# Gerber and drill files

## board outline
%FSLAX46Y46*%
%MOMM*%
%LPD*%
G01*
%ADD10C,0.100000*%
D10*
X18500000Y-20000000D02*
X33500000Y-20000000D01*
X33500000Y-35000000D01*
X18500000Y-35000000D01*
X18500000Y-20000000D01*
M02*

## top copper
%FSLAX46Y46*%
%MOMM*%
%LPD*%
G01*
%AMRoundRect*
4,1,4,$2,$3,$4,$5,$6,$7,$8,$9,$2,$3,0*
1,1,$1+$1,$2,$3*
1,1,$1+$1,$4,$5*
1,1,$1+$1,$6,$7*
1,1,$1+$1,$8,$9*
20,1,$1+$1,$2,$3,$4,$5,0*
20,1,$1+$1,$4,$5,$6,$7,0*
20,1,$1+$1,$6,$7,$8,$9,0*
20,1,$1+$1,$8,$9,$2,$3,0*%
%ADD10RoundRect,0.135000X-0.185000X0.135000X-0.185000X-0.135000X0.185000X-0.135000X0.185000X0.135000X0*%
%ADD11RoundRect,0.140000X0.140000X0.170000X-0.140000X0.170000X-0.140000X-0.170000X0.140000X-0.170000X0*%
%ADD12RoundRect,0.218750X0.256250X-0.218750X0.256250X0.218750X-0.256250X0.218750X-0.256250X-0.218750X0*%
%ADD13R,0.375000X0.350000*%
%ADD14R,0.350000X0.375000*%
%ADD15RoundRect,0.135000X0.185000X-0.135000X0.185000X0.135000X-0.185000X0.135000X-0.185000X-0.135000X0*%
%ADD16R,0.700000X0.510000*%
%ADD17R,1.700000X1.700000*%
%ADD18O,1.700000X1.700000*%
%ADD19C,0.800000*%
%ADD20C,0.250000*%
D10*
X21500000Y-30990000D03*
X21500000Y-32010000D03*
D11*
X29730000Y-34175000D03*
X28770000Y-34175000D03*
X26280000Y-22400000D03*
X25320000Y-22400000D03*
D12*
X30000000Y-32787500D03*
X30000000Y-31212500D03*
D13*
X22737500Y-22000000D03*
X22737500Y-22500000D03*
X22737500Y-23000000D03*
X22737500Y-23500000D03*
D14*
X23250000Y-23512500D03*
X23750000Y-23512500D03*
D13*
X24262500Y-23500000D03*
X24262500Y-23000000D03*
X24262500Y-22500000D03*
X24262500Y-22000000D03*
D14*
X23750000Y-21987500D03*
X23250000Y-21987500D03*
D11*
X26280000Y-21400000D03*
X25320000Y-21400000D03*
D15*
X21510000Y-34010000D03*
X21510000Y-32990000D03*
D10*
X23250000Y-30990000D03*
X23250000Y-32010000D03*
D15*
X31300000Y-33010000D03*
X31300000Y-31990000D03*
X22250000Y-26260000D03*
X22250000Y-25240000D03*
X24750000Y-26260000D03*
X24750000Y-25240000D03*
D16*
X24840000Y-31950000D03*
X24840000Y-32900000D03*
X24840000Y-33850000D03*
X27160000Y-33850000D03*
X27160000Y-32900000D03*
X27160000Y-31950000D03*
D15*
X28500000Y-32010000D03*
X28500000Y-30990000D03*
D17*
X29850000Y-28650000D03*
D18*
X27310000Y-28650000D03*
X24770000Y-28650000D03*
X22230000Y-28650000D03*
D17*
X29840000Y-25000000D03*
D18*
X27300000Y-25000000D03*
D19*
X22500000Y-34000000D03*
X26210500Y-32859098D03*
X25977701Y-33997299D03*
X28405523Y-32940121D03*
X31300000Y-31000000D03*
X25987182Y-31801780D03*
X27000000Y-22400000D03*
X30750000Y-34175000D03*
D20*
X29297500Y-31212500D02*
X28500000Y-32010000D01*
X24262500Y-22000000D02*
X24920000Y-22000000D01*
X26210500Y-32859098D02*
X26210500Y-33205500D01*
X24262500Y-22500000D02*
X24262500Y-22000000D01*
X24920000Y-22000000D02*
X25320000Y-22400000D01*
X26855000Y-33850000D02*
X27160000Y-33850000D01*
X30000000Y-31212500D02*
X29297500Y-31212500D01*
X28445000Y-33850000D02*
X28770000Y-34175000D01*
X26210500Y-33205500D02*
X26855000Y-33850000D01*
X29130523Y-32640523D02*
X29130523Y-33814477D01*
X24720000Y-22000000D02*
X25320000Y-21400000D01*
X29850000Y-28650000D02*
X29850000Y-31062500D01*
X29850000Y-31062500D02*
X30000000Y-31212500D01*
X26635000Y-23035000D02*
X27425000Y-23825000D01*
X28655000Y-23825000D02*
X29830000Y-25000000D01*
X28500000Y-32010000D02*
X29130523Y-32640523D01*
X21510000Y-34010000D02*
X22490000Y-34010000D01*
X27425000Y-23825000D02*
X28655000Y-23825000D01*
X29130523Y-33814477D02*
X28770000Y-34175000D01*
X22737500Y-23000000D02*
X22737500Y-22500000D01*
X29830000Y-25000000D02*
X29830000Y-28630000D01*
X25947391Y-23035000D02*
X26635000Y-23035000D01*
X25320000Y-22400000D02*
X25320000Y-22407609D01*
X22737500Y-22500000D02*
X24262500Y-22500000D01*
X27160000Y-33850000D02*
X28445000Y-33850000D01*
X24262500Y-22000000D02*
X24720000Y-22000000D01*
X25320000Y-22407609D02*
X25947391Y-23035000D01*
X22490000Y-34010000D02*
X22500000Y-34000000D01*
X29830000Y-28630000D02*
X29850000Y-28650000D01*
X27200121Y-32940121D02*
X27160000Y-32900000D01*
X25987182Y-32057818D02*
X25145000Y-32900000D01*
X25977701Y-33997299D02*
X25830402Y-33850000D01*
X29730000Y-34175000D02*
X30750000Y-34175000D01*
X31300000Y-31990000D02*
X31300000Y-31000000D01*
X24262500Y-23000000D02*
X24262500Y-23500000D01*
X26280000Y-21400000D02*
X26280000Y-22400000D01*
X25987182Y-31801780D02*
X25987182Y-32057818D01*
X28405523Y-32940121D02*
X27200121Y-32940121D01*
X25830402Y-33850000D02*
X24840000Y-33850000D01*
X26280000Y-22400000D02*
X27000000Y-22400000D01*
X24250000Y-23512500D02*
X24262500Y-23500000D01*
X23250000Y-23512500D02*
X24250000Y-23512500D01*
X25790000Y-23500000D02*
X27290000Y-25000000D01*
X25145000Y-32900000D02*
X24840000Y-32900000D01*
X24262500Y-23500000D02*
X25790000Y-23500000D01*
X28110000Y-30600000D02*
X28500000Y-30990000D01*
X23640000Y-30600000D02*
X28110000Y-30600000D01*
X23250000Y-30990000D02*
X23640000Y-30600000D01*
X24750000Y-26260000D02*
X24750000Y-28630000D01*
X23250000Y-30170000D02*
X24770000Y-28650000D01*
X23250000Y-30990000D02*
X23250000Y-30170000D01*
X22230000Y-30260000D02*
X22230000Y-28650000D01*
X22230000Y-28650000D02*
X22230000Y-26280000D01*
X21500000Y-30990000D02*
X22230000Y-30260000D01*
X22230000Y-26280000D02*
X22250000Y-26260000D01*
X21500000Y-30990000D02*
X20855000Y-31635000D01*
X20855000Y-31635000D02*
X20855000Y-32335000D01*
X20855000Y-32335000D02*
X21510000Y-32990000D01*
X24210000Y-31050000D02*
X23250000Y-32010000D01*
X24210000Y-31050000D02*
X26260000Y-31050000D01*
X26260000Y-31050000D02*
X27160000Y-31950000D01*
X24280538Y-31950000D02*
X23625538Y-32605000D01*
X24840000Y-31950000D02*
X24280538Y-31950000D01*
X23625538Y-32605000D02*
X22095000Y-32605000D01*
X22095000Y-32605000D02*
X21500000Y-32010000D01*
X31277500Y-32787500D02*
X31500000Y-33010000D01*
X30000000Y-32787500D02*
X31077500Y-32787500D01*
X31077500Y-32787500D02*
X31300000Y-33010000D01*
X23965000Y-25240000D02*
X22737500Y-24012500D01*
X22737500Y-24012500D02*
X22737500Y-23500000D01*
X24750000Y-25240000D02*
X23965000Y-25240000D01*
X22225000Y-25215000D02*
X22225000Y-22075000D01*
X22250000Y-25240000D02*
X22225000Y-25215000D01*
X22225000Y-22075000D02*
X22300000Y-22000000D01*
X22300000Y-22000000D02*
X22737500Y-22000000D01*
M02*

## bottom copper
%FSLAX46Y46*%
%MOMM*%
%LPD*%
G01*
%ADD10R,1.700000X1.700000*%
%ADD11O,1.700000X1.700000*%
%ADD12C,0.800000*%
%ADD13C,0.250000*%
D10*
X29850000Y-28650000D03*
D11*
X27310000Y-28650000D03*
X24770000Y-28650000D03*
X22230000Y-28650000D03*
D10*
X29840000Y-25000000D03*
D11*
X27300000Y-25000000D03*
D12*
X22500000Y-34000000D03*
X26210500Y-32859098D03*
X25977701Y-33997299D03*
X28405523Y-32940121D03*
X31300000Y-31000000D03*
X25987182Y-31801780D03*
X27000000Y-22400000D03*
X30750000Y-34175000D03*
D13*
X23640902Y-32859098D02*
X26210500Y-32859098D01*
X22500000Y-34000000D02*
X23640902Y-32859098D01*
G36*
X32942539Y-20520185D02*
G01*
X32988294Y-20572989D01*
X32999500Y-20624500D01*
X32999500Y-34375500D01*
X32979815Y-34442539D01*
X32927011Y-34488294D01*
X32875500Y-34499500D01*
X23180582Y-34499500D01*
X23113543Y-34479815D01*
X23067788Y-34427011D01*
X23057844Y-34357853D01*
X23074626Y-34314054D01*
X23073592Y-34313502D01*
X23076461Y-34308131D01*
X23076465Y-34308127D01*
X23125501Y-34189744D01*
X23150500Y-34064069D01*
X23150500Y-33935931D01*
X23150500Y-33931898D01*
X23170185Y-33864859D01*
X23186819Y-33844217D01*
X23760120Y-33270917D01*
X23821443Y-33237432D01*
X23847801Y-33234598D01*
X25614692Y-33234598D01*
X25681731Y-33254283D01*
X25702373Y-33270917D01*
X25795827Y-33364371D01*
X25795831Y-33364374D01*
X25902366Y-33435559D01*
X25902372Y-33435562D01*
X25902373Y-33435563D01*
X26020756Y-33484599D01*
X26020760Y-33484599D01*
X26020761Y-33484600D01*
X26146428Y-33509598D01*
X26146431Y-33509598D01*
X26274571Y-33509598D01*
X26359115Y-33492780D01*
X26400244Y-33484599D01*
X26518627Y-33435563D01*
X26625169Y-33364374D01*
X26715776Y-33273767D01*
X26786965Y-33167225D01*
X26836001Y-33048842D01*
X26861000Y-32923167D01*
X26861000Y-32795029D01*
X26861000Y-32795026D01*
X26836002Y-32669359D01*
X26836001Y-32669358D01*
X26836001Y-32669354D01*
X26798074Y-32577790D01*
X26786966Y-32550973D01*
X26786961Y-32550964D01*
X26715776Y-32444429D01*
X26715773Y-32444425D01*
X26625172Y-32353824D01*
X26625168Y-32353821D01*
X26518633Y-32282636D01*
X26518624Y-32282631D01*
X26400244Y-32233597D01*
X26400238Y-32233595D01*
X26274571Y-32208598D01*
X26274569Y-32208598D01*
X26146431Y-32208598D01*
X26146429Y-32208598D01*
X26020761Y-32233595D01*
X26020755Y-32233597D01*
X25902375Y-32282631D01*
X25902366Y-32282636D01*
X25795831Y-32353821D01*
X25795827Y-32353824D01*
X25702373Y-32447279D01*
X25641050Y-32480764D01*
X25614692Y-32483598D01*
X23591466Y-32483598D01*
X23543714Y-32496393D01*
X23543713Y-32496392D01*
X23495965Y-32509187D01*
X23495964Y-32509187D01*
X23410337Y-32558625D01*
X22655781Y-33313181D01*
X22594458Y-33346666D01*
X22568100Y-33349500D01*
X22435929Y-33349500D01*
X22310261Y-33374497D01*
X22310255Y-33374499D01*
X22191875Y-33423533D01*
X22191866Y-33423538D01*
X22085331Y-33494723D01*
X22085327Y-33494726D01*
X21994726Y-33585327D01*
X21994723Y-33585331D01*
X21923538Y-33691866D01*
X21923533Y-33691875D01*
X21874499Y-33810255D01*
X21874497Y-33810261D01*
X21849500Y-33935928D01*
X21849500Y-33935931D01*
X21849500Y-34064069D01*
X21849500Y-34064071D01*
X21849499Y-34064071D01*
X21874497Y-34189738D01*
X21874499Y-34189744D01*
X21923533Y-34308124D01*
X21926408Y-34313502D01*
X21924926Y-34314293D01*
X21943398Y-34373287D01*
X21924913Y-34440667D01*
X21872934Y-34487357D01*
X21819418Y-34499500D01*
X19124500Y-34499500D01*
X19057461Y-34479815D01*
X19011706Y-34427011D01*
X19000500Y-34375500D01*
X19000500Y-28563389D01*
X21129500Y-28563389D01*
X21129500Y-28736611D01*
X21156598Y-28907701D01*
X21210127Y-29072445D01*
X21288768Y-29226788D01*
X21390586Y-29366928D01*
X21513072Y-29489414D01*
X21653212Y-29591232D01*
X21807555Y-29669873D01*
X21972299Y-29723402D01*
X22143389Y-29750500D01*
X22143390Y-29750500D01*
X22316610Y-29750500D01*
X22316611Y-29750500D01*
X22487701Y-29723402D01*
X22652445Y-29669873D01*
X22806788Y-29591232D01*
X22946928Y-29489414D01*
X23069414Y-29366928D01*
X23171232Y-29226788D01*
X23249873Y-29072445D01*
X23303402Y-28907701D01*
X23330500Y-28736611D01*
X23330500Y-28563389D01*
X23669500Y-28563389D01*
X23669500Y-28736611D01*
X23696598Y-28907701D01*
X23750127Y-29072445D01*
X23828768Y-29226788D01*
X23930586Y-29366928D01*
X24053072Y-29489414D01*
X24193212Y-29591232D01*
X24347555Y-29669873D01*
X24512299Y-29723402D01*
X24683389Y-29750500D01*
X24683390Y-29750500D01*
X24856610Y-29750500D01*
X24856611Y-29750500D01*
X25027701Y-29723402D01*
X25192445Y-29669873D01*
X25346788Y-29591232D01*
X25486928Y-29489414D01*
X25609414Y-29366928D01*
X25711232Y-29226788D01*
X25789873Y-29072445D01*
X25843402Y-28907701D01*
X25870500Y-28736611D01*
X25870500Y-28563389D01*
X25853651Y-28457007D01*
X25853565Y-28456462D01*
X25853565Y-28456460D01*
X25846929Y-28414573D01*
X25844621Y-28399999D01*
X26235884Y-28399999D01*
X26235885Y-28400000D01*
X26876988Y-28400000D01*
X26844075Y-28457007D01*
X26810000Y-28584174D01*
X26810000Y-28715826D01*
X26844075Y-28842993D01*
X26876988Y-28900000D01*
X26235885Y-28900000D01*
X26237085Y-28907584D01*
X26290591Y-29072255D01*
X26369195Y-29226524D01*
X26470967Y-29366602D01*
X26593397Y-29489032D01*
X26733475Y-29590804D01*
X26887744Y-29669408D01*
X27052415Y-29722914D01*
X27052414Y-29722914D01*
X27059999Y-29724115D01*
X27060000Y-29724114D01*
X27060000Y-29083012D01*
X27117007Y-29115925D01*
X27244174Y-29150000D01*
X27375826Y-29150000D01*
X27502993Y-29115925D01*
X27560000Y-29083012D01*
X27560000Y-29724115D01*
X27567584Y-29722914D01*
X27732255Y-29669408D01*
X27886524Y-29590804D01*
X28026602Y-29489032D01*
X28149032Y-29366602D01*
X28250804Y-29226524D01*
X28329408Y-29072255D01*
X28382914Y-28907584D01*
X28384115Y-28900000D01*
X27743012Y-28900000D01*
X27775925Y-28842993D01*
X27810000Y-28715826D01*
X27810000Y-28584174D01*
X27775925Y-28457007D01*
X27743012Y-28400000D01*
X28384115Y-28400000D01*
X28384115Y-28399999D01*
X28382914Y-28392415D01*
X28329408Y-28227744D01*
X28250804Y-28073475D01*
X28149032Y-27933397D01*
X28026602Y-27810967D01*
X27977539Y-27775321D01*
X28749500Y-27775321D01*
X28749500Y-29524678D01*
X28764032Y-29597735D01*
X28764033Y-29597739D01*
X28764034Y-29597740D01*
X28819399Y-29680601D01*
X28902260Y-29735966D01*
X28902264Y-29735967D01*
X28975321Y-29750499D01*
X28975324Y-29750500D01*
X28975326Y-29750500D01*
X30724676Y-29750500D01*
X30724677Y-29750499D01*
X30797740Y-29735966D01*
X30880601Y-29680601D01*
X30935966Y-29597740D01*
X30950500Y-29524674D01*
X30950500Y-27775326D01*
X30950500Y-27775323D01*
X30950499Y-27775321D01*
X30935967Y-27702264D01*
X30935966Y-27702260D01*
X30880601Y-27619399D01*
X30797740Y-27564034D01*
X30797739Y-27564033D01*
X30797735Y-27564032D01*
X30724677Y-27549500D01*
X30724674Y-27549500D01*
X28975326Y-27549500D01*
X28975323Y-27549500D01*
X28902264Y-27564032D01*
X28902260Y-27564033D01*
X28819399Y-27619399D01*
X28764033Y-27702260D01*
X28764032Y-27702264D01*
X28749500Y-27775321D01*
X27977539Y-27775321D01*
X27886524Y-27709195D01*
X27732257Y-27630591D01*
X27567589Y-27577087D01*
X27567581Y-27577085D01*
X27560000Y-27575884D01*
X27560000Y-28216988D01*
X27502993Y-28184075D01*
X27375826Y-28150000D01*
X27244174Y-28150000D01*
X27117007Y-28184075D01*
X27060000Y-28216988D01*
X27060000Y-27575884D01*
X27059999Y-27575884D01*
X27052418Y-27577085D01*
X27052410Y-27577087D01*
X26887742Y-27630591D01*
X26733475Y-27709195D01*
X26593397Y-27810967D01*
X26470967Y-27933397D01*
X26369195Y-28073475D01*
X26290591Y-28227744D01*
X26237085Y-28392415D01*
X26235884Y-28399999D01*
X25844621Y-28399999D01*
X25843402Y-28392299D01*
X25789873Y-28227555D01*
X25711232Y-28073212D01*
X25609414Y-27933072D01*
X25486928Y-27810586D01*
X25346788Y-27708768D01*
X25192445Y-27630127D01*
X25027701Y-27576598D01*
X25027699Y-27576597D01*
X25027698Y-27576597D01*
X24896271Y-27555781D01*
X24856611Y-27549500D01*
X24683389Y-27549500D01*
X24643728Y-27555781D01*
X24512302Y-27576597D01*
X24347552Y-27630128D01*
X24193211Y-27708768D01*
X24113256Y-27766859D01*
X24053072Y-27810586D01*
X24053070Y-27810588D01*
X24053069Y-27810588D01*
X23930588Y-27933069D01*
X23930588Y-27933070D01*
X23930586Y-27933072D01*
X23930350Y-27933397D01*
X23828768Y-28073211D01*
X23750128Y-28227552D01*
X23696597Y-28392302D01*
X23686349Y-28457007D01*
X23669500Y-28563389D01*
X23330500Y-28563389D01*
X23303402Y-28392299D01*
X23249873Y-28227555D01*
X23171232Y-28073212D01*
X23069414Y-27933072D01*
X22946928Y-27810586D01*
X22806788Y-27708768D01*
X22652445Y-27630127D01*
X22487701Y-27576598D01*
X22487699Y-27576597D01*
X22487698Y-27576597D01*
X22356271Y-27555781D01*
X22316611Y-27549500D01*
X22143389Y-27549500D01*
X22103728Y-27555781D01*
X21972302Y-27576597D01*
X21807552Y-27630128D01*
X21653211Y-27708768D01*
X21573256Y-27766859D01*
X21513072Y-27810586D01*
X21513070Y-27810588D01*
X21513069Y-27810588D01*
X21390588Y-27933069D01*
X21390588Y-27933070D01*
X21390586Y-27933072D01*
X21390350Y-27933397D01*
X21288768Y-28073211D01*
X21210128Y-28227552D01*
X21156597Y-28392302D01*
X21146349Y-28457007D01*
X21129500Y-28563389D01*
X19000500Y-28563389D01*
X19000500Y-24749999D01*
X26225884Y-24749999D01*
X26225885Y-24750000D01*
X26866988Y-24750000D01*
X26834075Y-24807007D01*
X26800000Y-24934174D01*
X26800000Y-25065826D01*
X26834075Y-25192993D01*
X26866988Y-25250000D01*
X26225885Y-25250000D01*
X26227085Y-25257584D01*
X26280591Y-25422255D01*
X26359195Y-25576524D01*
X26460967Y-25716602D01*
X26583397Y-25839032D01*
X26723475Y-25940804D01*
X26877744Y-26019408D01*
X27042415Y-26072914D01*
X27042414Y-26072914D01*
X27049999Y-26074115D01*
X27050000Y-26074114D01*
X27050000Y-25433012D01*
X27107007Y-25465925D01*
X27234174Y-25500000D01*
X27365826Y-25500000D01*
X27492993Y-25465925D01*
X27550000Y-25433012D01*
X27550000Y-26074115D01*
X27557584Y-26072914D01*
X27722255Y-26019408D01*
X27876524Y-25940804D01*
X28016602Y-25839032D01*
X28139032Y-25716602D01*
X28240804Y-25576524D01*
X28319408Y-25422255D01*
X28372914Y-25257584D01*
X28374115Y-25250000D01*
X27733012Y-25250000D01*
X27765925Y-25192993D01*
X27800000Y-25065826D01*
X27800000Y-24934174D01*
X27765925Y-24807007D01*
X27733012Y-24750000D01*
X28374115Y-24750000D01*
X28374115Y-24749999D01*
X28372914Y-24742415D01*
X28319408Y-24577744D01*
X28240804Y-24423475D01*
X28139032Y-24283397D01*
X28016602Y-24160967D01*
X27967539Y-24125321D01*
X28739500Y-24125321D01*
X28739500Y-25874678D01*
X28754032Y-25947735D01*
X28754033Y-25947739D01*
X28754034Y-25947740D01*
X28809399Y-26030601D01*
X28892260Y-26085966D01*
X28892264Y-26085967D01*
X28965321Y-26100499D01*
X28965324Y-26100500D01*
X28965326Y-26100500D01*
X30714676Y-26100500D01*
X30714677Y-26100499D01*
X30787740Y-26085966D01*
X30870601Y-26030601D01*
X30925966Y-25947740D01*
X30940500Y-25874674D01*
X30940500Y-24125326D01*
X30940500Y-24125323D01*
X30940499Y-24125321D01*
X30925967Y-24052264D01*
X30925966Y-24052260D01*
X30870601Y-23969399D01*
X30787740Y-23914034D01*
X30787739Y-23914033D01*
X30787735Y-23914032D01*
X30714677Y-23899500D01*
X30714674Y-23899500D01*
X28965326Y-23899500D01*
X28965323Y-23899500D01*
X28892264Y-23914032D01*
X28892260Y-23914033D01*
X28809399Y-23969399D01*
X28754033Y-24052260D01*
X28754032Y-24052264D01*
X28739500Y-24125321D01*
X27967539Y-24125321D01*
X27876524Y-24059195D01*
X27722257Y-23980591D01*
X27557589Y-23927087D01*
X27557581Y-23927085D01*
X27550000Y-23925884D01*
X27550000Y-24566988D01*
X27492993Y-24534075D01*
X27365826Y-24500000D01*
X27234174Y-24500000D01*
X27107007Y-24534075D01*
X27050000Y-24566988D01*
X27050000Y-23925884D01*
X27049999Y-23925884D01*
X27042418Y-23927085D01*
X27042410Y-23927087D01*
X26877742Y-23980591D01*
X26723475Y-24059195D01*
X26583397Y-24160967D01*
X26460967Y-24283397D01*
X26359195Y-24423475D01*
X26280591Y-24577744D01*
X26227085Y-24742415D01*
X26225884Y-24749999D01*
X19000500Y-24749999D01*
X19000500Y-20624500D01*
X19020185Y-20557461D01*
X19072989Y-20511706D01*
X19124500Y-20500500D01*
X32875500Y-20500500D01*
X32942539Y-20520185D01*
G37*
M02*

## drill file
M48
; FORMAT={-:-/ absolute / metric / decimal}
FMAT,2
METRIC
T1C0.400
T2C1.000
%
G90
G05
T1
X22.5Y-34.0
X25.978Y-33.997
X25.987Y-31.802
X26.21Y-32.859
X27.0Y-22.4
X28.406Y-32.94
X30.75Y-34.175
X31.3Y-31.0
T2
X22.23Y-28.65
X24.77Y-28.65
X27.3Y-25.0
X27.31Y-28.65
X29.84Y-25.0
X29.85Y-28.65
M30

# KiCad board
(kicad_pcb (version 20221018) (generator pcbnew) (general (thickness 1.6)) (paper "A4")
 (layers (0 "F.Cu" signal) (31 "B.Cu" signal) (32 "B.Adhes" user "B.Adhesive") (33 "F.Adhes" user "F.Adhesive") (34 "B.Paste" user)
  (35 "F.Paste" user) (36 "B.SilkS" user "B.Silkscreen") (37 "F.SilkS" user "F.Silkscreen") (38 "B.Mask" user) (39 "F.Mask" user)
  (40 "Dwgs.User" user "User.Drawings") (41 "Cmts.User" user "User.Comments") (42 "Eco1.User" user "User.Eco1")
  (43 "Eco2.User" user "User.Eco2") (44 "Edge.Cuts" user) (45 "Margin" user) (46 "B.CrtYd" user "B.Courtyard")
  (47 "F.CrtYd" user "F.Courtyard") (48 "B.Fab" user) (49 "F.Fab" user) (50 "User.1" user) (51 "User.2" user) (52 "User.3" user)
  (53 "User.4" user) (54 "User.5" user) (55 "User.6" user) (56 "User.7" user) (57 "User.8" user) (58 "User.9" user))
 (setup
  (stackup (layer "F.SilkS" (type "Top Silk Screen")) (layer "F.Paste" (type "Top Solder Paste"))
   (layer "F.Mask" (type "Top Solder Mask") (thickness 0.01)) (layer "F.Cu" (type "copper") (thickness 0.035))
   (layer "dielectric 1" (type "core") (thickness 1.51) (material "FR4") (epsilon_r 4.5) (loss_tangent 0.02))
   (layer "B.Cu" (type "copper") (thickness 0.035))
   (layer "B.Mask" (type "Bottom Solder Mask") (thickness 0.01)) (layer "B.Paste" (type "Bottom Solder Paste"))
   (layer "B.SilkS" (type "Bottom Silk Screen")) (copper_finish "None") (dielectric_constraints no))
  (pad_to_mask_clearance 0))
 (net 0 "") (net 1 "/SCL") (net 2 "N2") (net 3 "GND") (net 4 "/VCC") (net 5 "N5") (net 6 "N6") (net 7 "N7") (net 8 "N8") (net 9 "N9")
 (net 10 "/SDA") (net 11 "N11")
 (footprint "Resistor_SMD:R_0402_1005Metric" (layer "F.Cu") (at 21.5 31.5 -90)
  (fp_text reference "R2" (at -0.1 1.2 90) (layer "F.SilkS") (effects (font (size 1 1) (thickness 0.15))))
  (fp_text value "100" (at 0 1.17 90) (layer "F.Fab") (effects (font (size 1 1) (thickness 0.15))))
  (pad "1" smd roundrect (at -0.51 0 270) (size 0.54 0.64) (layers "F.Cu" "F.Paste" "F.Mask") (roundrect_rratio 0.25) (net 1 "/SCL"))
  (pad "2" smd roundrect (at 0.51 0 270) (size 0.54 0.64) (layers "F.Cu" "F.Paste" "F.Mask") (roundrect_rratio 0.25) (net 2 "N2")))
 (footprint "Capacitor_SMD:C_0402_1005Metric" (layer "F.Cu") (at 29.25 34.175 180)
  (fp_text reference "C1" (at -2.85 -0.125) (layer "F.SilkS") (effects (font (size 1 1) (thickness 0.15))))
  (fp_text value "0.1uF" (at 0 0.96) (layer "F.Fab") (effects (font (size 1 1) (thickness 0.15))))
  (pad "1" smd roundrect (at -0.48 0 180) (size 0.56 0.62) (layers "F.Cu" "F.Paste" "F.Mask") (roundrect_rratio 0.25) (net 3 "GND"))
  (pad "2" smd roundrect (at 0.48 0 180) (size 0.56 0.62) (layers "F.Cu" "F.Paste" "F.Mask") (roundrect_rratio 0.25) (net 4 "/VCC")))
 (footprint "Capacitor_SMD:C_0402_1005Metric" (layer "F.Cu") (at 25.8 22.4 180)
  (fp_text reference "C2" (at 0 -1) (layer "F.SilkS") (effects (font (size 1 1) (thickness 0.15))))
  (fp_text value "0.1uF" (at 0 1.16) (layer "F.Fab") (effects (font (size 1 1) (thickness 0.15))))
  (pad "1" smd roundrect (at -0.48 0 180) (size 0.56 0.62) (layers "F.Cu" "F.Paste" "F.Mask") (roundrect_rratio 0.25) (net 3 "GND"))
  (pad "2" smd roundrect (at 0.48 0 180) (size 0.56 0.62) (layers "F.Cu" "F.Paste" "F.Mask") (roundrect_rratio 0.25) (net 4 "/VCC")))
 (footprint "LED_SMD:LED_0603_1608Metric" (layer "F.Cu") (at 30 32 90)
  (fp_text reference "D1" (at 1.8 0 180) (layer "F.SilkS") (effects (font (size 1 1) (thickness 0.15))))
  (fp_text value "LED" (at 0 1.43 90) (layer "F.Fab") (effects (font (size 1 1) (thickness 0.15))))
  (pad "1" smd roundrect (at -0.7875 0 90) (size 0.875 0.95) (layers "F.Cu" "F.Paste" "F.Mask") (roundrect_rratio 0.25) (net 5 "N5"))
  (pad "2" smd roundrect (at 0.7875 0 90) (size 0.875 0.95) (layers "F.Cu" "F.Paste" "F.Mask") (roundrect_rratio 0.25) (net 4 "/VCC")))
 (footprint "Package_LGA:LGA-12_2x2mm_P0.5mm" (layer "F.Cu") (at 23.5 22.75)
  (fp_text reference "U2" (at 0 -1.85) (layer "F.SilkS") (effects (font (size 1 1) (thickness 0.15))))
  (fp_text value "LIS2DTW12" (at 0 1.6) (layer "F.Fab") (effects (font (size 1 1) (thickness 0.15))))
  (pad "1" smd rect (at -0.7625 -0.75) (size 0.375 0.35) (layers "F.Cu" "F.Paste" "F.Mask") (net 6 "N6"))
  (pad "2" smd rect (at -0.7625 -0.25) (size 0.375 0.35) (layers "F.Cu" "F.Paste" "F.Mask") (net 4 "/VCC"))
  (pad "3" smd rect (at -0.7625 0.25) (size 0.375 0.35) (layers "F.Cu" "F.Paste" "F.Mask") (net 4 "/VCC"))
  (pad "4" smd rect (at -0.7625 0.75) (size 0.375 0.35) (layers "F.Cu" "F.Paste" "F.Mask") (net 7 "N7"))
  (pad "5" smd rect (at -0.25 0.7625 90) (size 0.375 0.35) (layers "F.Cu" "F.Paste" "F.Mask") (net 3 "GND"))
  (pad "6" smd rect (at 0.25 0.7625 90) (size 0.375 0.35) (layers "F.Cu" "F.Paste" "F.Mask") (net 3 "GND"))
  (pad "7" smd rect (at 0.7625 0.75) (size 0.375 0.35) (layers "F.Cu" "F.Paste" "F.Mask") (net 3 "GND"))
  (pad "8" smd rect (at 0.7625 0.25) (size 0.375 0.35) (layers "F.Cu" "F.Paste" "F.Mask") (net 3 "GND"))
  (pad "9" smd rect (at 0.7625 -0.25) (size 0.375 0.35) (layers "F.Cu" "F.Paste" "F.Mask") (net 4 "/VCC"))
  (pad "10" smd rect (at 0.7625 -0.75) (size 0.375 0.35) (layers "F.Cu" "F.Paste" "F.Mask") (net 4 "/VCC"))
  (pad "11" smd rect (at 0.25 -0.7625 90) (size 0.375 0.35) (layers "F.Cu" "F.Paste" "F.Mask") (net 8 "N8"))
  (pad "12" smd rect (at -0.25 -0.7625 90) (size 0.375 0.35) (layers "F.Cu" "F.Paste" "F.Mask") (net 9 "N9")))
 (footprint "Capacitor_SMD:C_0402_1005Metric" (layer "F.Cu") (at 25.8 21.4 180)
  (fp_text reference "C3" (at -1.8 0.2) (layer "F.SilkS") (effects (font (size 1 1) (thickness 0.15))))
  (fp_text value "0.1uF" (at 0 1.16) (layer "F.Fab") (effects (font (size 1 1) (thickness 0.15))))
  (pad "1" smd roundrect (at -0.48 0 180) (size 0.56 0.62) (layers "F.Cu" "F.Paste" "F.Mask") (roundrect_rratio 0.25) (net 3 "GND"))
  (pad "2" smd roundrect (at 0.48 0 180) (size 0.56 0.62) (layers "F.Cu" "F.Paste" "F.Mask") (roundrect_rratio 0.25) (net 4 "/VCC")))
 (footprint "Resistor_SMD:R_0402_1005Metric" (layer "F.Cu") (at 21.51 33.5 90)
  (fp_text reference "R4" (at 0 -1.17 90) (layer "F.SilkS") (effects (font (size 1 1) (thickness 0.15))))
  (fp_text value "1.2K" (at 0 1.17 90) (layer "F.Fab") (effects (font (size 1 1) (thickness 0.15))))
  (pad "1" smd roundrect (at -0.51 0 90) (size 0.54 0.64) (layers "F.Cu" "F.Paste" "F.Mask") (roundrect_rratio 0.25) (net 4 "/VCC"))
  (pad "2" smd roundrect (at 0.51 0 90) (size 0.54 0.64) (layers "F.Cu" "F.Paste" "F.Mask") (roundrect_rratio 0.25) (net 1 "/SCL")))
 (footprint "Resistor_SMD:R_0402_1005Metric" (layer "F.Cu") (at 23.25 31.5 -90)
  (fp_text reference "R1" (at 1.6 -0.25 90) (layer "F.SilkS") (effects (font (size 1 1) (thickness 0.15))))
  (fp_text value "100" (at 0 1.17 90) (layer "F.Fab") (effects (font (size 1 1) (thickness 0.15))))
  (pad "1" smd roundrect (at -0.51 0 270) (size 0.54 0.64) (layers "F.Cu" "F.Paste" "F.Mask") (roundrect_rratio 0.25) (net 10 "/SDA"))
  (pad "2" smd roundrect (at 0.51 0 270) (size 0.54 0.64) (layers "F.Cu" "F.Paste" "F.Mask") (roundrect_rratio 0.25) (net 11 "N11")))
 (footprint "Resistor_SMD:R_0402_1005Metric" (layer "F.Cu") (at 31.3 32.5 90)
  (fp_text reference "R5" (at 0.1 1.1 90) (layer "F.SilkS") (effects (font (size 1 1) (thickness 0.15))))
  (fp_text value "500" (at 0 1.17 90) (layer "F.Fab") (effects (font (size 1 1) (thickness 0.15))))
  (pad "1" smd roundrect (at -0.51 0 90) (size 0.54 0.64) (layers "F.Cu" "F.Paste" "F.Mask") (roundrect_rratio 0.25) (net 5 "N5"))
  (pad "2" smd roundrect (at 0.51 0 90) (size 0.54 0.64) (layers "F.Cu" "F.Paste" "F.Mask") (roundrect_rratio 0.25) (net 3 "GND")))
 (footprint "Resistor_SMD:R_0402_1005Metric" (layer "F.Cu") (at 22.25 25.75 90)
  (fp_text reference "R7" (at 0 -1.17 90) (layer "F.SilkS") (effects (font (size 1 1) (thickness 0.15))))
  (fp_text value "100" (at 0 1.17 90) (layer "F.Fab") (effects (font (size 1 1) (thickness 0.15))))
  (pad "1" smd roundrect (at -0.51 0 90) (size 0.54 0.64) (layers "F.Cu" "F.Paste" "F.Mask") (roundrect_rratio 0.25) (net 1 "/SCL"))
  (pad "2" smd roundrect (at 0.51 0 90) (size 0.54 0.64) (layers "F.Cu" "F.Paste" "F.Mask") (roundrect_rratio 0.25) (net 6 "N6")))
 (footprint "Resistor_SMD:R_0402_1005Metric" (layer "F.Cu") (at 24.75 25.75 90)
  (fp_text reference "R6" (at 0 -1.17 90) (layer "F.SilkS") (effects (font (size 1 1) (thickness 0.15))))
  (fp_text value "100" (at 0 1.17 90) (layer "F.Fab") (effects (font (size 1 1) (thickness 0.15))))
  (pad "1" smd roundrect (at -0.51 0 90) (size 0.54 0.64) (layers "F.Cu" "F.Paste" "F.Mask") (roundrect_rratio 0.25) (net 10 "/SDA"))
  (pad "2" smd roundrect (at 0.51 0 90) (size 0.54 0.64) (layers "F.Cu" "F.Paste" "F.Mask") (roundrect_rratio 0.25) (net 7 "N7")))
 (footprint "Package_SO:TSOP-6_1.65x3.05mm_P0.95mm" (layer "F.Cu") (at 26 32.9)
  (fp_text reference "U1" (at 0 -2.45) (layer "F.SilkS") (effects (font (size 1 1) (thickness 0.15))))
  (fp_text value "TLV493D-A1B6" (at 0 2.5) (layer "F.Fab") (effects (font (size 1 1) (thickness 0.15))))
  (pad "1" smd rect (at -1.16 -0.95) (size 0.7 0.51) (layers "F.Cu" "F.Paste" "F.Mask") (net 2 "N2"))
  (pad "2" smd rect (at -1.16 0) (size 0.7 0.51) (layers "F.Cu" "F.Paste" "F.Mask") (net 3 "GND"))
  (pad "3" smd rect (at -1.16 0.95) (size 0.7 0.51) (layers "F.Cu" "F.Paste" "F.Mask") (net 3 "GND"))
  (pad "4" smd rect (at 1.16 0.95) (size 0.7 0.51) (layers "F.Cu" "F.Paste" "F.Mask") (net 4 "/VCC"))
  (pad "5" smd rect (at 1.16 0) (size 0.7 0.51) (layers "F.Cu" "F.Paste" "F.Mask") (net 3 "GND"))
  (pad "6" smd rect (at 1.16 -0.95) (size 0.7 0.51) (layers "F.Cu" "F.Paste" "F.Mask") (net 11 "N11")))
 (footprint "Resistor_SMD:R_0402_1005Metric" (layer "F.Cu") (at 28.5 31.5 90)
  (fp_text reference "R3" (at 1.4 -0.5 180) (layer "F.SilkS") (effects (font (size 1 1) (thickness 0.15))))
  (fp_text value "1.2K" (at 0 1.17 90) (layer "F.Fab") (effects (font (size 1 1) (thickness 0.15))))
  (pad "1" smd roundrect (at -0.51 0 90) (size 0.54 0.64) (layers "F.Cu" "F.Paste" "F.Mask") (roundrect_rratio 0.25) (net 4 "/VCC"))
  (pad "2" smd roundrect (at 0.51 0 90) (size 0.54 0.64) (layers "F.Cu" "F.Paste" "F.Mask") (roundrect_rratio 0.25) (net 10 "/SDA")))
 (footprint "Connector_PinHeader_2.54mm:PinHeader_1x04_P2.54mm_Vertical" (layer "B.Cu") (at 29.85 28.65 90)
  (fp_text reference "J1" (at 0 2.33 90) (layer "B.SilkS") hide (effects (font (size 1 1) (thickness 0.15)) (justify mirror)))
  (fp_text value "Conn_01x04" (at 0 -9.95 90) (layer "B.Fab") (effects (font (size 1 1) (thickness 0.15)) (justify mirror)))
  (pad "1" thru_hole rect (at 0 0 90) (size 1.7 1.7) (drill 1) (layers "*.Cu" "*.Mask") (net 4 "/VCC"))
  (pad "2" thru_hole oval (at 0 -2.54 90) (size 1.7 1.7) (drill 1) (layers "*.Cu" "*.Mask") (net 3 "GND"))
  (pad "3" thru_hole oval (at 0 -5.08 90) (size 1.7 1.7) (drill 1) (layers "*.Cu" "*.Mask") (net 10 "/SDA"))
  (pad "4" thru_hole oval (at 0 -7.62 90) (size 1.7 1.7) (drill 1) (layers "*.Cu" "*.Mask") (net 1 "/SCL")))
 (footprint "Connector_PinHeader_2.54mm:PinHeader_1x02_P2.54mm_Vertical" (layer "B.Cu") (at 29.84 25 90)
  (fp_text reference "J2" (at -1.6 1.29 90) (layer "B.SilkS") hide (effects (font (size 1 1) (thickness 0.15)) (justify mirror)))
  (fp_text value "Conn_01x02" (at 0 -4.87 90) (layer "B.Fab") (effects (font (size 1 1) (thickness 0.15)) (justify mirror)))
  (pad "1" thru_hole rect (at 0 0 90) (size 1.7 1.7) (drill 1) (layers "*.Cu" "*.Mask") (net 4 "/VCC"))
  (pad "2" thru_hole oval (at 0 -2.54 90) (size 1.7 1.7) (drill 1) (layers "*.Cu" "*.Mask") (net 3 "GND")))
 (gr_rect (start 18.5 20) (end 33.5 35) (stroke (width 0.1) (type default)) (fill none) (layer "Edge.Cuts"))
 (segment (start 29.2975 31.2125) (end 28.5 32.01) (width 0.25) (layer "F.Cu") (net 4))
 (segment (start 24.2625 22) (end 24.92 22) (width 0.25) (layer "F.Cu") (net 4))
 (segment (start 26.2105 32.859098) (end 26.2105 33.2055) (width 0.25) (layer "F.Cu") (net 4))
 (segment (start 24.2625 22.5) (end 24.2625 22) (width 0.25) (layer "F.Cu") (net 4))
 (segment (start 24.92 22) (end 25.32 22.4) (width 0.25) (layer "F.Cu") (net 4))
 (segment (start 26.855 33.85) (end 27.16 33.85) (width 0.25) (layer "F.Cu") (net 4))
 (segment (start 30 31.2125) (end 29.2975 31.2125) (width 0.25) (layer "F.Cu") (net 4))
 (segment (start 28.445 33.85) (end 28.77 34.175) (width 0.25) (layer "F.Cu") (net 4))
 (segment (start 26.2105 33.2055) (end 26.855 33.85) (width 0.25) (layer "F.Cu") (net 4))
 (segment (start 29.130523 32.640523) (end 29.130523 33.814477) (width 0.25) (layer "F.Cu") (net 4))
 (segment (start 24.72 22) (end 25.32 21.4) (width 0.25) (layer "F.Cu") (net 4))
 (segment (start 29.85 28.65) (end 29.85 31.0625) (width 0.25) (layer "F.Cu") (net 4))
 (segment (start 29.85 31.0625) (end 30 31.2125) (width 0.25) (layer "F.Cu") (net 4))
 (segment (start 26.635 23.035) (end 27.425 23.825) (width 0.25) (layer "F.Cu") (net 4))
 (segment (start 28.655 23.825) (end 29.83 25) (width 0.25) (layer "F.Cu") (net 4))
 (segment (start 28.5 32.01) (end 29.130523 32.640523) (width 0.25) (layer "F.Cu") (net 4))
 (segment (start 21.51 34.01) (end 22.49 34.01) (width 0.25) (layer "F.Cu") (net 4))
 (segment (start 27.425 23.825) (end 28.655 23.825) (width 0.25) (layer "F.Cu") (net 4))
 (segment (start 29.130523 33.814477) (end 28.77 34.175) (width 0.25) (layer "F.Cu") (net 4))
 (segment (start 22.7375 23) (end 22.7375 22.5) (width 0.25) (layer "F.Cu") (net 4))
 (segment (start 29.83 25) (end 29.83 28.63) (width 0.25) (layer "F.Cu") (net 4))
 (segment (start 25.947391 23.035) (end 26.635 23.035) (width 0.25) (layer "F.Cu") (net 4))
 (segment (start 25.32 22.4) (end 25.32 22.407609) (width 0.25) (layer "F.Cu") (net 4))
 (segment (start 22.7375 22.5) (end 24.2625 22.5) (width 0.25) (layer "F.Cu") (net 4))
 (segment (start 27.16 33.85) (end 28.445 33.85) (width 0.25) (layer "F.Cu") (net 4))
 (segment (start 24.2625 22) (end 24.72 22) (width 0.25) (layer "F.Cu") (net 4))
 (segment (start 25.32 22.407609) (end 25.947391 23.035) (width 0.25) (layer "F.Cu") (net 4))
 (segment (start 22.49 34.01) (end 22.5 34) (width 0.25) (layer "F.Cu") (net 4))
 (segment (start 29.83 28.63) (end 29.85 28.65) (width 0.25) (layer "F.Cu") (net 4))
 (via (at 22.5 34) (size 0.8) (drill 0.4) (layers "F.Cu" "B.Cu") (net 4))
 (via (at 26.2105 32.859098) (size 0.8) (drill 0.4) (layers "F.Cu" "B.Cu") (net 4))
 (segment (start 23.640902 32.859098) (end 26.2105 32.859098) (width 0.25) (layer "B.Cu") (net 4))
 (segment (start 22.5 34) (end 23.640902 32.859098) (width 0.25) (layer "B.Cu") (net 4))
 (segment (start 27.200121 32.940121) (end 27.16 32.9) (width 0.25) (layer "F.Cu") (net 3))
 (segment (start 25.987182 32.057818) (end 25.145 32.9) (width 0.25) (layer "F.Cu") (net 3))
 (segment (start 25.977701 33.997299) (end 25.830402 33.85) (width 0.25) (layer "F.Cu") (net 3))
 (segment (start 29.73 34.175) (end 30.75 34.175) (width 0.25) (layer "F.Cu") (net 3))
 (segment (start 31.3 31.99) (end 31.3 31) (width 0.25) (layer "F.Cu") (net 3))
 (segment (start 24.2625 23) (end 24.2625 23.5) (width 0.25) (layer "F.Cu") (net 3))
 (segment (start 26.28 21.4) (end 26.28 22.4) (width 0.25) (layer "F.Cu") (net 3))
 (segment (start 25.987182 31.80178) (end 25.987182 32.057818) (width 0.25) (layer "F.Cu") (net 3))
 (segment (start 28.405523 32.940121) (end 27.200121 32.940121) (width 0.25) (layer "F.Cu") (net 3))
 (segment (start 25.830402 33.85) (end 24.84 33.85) (width 0.25) (layer "F.Cu") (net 3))
 (segment (start 26.28 22.4) (end 27 22.4) (width 0.25) (layer "F.Cu") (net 3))
 (segment (start 24.25 23.5125) (end 24.2625 23.5) (width 0.25) (layer "F.Cu") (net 3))
 (segment (start 23.25 23.5125) (end 24.25 23.5125) (width 0.25) (layer "F.Cu") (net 3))
 (segment (start 25.79 23.5) (end 27.29 25) (width 0.25) (layer "F.Cu") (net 3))
 (segment (start 25.145 32.9) (end 24.84 32.9) (width 0.25) (layer "F.Cu") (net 3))
 (segment (start 24.2625 23.5) (end 25.79 23.5) (width 0.25) (layer "F.Cu") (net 3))
 (via (at 25.977701 33.997299) (size 0.8) (drill 0.4) (layers "F.Cu" "B.Cu") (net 3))
 (via (at 28.405523 32.940121) (size 0.8) (drill 0.4) (layers "F.Cu" "B.Cu") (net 3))
 (via (at 31.3 31) (size 0.8) (drill 0.4) (layers "F.Cu" "B.Cu") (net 3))
 (via (at 25.987182 31.80178) (size 0.8) (drill 0.4) (layers "F.Cu" "B.Cu") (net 3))
 (via (at 27 22.4) (size 0.8) (drill 0.4) (layers "F.Cu" "B.Cu") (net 3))
 (via (at 30.75 34.175) (size 0.8) (drill 0.4) (layers "F.Cu" "B.Cu") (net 3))
 (segment (start 28.11 30.6) (end 28.5 30.99) (width 0.25) (layer "F.Cu") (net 10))
 (segment (start 23.64 30.6) (end 28.11 30.6) (width 0.25) (layer "F.Cu") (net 10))
 (segment (start 23.25 30.99) (end 23.64 30.6) (width 0.25) (layer "F.Cu") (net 10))
 (segment (start 24.75 26.26) (end 24.75 28.63) (width 0.25) (layer "F.Cu") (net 10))
 (segment (start 23.25 30.17) (end 24.77 28.65) (width 0.25) (layer "F.Cu") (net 10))
 (segment (start 23.25 30.99) (end 23.25 30.17) (width 0.25) (layer "F.Cu") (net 10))
 (segment (start 22.23 30.26) (end 22.23 28.65) (width 0.25) (layer "F.Cu") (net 1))
 (segment (start 22.23 28.65) (end 22.23 26.28) (width 0.25) (layer "F.Cu") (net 1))
 (segment (start 21.5 30.99) (end 22.23 30.26) (width 0.25) (layer "F.Cu") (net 1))
 (segment (start 22.23 26.28) (end 22.25 26.26) (width 0.25) (layer "F.Cu") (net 1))
 (segment (start 21.5 30.99) (end 20.855 31.635) (width 0.25) (layer "F.Cu") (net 1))
 (segment (start 20.855 31.635) (end 20.855 32.335) (width 0.25) (layer "F.Cu") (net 1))
 (segment (start 20.855 32.335) (end 21.51 32.99) (width 0.25) (layer "F.Cu") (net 1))
 (segment (start 24.21 31.05) (end 23.25 32.01) (width 0.25) (layer "F.Cu") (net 11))
 (segment (start 24.21 31.05) (end 26.26 31.05) (width 0.25) (layer "F.Cu") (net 11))
 (segment (start 26.26 31.05) (end 27.16 31.95) (width 0.25) (layer "F.Cu") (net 11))
 (segment (start 24.280538 31.95) (end 23.625538 32.605) (width 0.25) (layer "F.Cu") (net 2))
 (segment (start 24.84 31.95) (end 24.280538 31.95) (width 0.25) (layer "F.Cu") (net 2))
 (segment (start 23.625538 32.605) (end 22.095 32.605) (width 0.25) (layer "F.Cu") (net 2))
 (segment (start 22.095 32.605) (end 21.5 32.01) (width 0.25) (layer "F.Cu") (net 2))
 (segment (start 31.2775 32.7875) (end 31.5 33.01) (width 0.25) (layer "F.Cu") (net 5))
 (segment (start 30 32.7875) (end 31.0775 32.7875) (width 0.25) (layer "F.Cu") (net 5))
 (segment (start 31.0775 32.7875) (end 31.3 33.01) (width 0.25) (layer "F.Cu") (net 5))
 (segment (start 23.965 25.24) (end 22.7375 24.0125) (width 0.25) (layer "F.Cu") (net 7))
 (segment (start 22.7375 24.0125) (end 22.7375 23.5) (width 0.25) (layer "F.Cu") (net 7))
 (segment (start 24.75 25.24) (end 23.965 25.24) (width 0.25) (layer "F.Cu") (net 7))
 (segment (start 22.225 25.215) (end 22.225 22.075) (width 0.25) (layer "F.Cu") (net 6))
 (segment (start 22.25 25.24) (end 22.225 25.215) (width 0.25) (layer "F.Cu") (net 6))
 (segment (start 22.225 22.075) (end 22.3 22) (width 0.25) (layer "F.Cu") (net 6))
 (segment (start 22.3 22) (end 22.7375 22) (width 0.25) (layer "F.Cu") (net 6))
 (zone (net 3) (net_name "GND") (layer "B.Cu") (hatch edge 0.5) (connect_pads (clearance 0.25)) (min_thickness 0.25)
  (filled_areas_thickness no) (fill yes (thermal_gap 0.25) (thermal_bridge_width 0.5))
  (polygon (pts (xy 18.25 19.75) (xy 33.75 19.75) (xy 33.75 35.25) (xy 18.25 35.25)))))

